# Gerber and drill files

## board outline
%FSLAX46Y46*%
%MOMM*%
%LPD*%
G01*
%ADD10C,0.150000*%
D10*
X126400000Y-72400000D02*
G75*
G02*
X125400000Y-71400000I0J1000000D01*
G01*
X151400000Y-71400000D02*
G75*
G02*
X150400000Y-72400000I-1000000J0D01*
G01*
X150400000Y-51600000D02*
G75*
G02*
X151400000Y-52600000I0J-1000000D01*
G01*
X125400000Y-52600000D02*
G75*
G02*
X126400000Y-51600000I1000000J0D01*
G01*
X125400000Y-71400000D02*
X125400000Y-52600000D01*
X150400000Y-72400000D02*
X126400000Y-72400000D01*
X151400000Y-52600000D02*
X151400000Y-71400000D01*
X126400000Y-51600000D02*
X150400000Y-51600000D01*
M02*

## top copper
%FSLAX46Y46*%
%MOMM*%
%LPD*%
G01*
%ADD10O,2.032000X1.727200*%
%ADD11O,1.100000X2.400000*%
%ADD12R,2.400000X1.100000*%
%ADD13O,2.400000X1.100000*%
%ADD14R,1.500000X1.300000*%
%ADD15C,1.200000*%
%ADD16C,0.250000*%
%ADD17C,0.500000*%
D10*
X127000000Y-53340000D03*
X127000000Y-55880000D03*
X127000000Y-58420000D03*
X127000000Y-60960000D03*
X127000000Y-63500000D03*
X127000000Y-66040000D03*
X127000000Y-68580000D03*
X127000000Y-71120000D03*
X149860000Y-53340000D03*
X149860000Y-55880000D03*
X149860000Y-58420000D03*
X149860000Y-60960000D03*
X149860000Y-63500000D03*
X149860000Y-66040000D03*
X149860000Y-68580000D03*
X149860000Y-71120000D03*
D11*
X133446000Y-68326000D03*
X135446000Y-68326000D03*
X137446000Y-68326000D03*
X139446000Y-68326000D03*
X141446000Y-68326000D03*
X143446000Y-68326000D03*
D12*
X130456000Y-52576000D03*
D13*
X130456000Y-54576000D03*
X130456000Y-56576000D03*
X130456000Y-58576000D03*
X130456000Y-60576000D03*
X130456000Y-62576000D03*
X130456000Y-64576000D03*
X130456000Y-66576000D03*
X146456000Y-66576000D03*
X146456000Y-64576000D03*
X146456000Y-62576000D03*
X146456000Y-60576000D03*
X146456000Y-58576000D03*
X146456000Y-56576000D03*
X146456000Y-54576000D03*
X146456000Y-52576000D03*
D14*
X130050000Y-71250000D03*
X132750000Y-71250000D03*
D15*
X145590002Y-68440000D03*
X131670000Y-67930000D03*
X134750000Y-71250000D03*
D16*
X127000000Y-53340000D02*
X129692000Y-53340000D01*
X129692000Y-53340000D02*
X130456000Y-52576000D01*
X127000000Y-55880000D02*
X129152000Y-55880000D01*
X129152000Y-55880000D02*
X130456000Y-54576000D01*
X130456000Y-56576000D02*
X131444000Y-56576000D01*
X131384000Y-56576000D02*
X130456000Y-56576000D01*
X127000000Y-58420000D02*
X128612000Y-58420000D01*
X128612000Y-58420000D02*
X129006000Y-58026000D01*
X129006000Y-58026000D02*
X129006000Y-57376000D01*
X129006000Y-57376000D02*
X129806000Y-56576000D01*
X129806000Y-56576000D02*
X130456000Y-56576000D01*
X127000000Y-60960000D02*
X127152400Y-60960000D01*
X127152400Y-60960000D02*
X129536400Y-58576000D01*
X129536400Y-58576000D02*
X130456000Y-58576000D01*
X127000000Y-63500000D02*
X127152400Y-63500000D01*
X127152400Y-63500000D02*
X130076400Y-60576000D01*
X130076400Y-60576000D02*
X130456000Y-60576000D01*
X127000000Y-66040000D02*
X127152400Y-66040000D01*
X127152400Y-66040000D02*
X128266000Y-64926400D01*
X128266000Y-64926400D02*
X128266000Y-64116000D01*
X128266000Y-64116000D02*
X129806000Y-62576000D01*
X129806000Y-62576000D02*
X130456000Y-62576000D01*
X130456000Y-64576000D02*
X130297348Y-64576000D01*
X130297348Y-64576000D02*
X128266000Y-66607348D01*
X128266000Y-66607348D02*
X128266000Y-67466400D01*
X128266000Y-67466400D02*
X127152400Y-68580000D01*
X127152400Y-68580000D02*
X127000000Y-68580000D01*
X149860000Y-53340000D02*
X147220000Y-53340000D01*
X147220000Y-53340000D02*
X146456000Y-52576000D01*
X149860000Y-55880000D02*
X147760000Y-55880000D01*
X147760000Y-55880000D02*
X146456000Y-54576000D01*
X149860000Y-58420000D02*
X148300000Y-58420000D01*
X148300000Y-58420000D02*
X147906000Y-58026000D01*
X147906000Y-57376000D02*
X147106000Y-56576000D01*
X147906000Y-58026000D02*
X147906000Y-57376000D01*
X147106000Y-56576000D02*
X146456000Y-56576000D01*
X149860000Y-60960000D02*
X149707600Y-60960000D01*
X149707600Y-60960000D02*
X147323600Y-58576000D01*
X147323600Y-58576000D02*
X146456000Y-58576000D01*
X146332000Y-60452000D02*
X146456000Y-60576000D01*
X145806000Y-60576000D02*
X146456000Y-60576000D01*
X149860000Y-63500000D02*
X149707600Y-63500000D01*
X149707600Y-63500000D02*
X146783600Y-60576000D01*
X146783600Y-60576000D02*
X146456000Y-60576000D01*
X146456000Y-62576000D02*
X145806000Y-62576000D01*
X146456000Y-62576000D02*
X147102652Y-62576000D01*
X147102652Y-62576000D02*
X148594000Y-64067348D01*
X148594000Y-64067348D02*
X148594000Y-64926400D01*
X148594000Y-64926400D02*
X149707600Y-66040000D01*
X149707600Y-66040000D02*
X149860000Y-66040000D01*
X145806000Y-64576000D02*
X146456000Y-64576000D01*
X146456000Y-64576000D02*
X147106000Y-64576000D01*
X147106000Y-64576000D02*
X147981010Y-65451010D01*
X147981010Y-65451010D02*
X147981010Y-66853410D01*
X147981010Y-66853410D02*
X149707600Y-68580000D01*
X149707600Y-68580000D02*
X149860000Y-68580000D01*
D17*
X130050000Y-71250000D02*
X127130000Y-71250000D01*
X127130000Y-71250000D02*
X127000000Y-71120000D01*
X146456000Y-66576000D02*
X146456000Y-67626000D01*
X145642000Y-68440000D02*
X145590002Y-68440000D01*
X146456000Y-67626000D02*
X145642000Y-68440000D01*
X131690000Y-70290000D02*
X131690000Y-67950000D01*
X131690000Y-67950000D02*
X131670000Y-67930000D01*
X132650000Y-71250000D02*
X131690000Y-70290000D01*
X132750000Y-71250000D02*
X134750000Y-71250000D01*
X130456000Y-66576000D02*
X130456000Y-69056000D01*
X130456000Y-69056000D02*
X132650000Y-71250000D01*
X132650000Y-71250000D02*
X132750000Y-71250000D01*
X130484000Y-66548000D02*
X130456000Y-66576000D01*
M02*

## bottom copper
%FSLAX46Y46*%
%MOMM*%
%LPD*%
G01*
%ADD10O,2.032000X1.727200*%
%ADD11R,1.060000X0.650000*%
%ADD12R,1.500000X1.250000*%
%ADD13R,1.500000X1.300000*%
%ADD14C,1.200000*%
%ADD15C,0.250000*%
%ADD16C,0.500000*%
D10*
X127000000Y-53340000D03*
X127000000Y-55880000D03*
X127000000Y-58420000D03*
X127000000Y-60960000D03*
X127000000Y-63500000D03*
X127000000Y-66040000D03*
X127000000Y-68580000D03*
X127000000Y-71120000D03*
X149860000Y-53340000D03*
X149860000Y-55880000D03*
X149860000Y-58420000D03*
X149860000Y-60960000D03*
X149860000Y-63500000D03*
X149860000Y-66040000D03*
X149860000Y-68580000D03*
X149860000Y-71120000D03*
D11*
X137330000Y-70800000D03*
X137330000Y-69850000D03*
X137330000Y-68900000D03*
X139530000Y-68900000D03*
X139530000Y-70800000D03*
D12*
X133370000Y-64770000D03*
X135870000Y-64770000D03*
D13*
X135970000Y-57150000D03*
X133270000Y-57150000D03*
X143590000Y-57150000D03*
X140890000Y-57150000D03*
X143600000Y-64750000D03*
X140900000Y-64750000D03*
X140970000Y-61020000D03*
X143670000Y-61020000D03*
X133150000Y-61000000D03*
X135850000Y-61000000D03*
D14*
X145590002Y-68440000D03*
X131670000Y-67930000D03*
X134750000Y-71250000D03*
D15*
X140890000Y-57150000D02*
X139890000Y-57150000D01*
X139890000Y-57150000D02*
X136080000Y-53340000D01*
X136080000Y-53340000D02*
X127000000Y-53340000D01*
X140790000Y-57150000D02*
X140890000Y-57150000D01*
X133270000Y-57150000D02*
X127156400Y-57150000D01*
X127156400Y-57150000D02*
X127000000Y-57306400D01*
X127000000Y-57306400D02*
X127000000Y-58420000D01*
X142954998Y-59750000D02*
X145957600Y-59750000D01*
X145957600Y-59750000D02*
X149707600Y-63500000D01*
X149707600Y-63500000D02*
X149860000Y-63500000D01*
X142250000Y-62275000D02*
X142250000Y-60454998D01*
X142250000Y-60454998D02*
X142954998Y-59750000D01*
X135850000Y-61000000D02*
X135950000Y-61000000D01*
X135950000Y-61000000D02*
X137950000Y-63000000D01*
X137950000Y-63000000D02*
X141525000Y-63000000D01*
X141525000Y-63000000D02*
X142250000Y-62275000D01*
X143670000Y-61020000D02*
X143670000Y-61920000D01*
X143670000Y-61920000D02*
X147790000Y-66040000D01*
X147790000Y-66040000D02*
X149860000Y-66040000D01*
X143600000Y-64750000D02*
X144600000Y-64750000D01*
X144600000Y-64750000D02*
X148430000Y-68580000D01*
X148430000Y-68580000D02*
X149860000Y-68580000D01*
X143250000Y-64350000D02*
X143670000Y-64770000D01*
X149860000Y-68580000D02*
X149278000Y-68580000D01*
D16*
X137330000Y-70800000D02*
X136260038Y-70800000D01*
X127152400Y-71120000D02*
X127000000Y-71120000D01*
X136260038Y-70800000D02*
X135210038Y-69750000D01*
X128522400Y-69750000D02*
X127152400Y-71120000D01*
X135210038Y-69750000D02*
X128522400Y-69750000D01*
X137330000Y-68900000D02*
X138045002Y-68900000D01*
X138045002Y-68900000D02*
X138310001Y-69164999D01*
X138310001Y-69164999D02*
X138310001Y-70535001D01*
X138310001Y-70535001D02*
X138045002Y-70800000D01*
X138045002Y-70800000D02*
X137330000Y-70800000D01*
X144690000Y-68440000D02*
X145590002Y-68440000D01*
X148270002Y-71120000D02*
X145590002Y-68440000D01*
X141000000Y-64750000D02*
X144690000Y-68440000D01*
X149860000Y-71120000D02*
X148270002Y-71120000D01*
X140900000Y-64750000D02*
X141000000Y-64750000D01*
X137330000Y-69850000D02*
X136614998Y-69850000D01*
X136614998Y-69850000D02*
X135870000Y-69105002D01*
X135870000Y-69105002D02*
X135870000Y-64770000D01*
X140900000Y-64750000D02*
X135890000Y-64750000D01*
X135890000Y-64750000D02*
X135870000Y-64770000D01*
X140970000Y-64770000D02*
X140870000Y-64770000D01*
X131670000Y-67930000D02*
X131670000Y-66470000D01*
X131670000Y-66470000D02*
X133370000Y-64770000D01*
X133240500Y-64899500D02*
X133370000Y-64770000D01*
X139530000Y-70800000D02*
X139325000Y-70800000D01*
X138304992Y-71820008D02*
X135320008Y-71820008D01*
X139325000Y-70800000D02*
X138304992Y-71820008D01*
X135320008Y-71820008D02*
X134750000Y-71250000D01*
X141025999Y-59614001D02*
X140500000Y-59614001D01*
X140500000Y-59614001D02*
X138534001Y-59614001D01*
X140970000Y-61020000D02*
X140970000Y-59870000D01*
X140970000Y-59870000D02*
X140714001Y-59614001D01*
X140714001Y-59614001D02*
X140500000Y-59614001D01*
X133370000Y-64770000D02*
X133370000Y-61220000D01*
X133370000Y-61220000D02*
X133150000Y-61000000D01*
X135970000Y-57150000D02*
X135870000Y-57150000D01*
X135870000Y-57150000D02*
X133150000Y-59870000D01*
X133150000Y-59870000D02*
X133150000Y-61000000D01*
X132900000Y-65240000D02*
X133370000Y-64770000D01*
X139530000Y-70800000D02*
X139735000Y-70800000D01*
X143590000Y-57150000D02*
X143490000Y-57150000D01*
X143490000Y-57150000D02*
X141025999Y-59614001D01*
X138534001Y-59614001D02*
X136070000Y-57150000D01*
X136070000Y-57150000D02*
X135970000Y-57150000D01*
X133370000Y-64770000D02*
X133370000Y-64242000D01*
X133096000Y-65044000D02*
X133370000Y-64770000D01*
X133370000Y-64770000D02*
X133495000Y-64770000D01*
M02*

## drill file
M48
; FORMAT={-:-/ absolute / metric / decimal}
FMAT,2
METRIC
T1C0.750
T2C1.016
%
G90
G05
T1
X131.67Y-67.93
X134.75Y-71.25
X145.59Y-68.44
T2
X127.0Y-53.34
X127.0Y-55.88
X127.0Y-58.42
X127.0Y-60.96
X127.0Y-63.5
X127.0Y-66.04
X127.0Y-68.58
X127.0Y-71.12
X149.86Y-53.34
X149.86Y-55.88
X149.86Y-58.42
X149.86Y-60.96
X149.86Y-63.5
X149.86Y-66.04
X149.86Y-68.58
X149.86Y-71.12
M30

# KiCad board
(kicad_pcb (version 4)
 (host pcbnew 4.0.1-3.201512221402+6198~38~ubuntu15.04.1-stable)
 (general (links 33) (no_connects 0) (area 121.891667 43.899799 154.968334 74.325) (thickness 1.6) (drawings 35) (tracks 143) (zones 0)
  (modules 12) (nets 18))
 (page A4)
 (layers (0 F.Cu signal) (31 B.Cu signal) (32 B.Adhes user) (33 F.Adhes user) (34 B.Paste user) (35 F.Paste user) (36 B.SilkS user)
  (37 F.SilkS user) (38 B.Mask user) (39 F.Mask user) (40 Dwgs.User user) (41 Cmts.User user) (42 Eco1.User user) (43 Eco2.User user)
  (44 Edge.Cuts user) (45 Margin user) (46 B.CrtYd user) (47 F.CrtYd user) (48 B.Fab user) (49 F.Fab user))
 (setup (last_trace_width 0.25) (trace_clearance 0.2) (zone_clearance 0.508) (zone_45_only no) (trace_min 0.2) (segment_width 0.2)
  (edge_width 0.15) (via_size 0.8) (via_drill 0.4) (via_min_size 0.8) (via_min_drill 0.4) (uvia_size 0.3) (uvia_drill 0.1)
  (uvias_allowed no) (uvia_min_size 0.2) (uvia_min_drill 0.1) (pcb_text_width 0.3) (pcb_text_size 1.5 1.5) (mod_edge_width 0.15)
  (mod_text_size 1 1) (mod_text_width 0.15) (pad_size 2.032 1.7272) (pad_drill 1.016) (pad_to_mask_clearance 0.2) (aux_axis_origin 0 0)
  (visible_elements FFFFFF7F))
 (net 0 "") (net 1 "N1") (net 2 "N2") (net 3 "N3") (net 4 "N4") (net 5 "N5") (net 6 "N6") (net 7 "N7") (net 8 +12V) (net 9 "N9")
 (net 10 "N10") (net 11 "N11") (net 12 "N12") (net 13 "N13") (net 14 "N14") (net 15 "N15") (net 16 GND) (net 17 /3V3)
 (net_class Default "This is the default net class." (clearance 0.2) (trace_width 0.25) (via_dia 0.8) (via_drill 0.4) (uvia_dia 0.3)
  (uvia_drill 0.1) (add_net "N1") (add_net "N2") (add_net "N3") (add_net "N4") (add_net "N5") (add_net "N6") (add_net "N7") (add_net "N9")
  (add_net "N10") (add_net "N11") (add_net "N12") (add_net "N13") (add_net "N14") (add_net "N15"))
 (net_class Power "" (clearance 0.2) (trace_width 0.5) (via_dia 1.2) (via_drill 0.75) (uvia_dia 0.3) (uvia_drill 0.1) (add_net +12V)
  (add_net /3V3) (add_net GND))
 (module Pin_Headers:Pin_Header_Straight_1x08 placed (layer B.Cu) (at 127 53.34 180)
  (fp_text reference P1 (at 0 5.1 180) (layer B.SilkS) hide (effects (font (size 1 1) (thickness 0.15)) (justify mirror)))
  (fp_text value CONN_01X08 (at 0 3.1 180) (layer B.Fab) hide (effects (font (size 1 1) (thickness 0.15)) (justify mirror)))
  (pad 1 thru_hole oval (at 0 0 180) (size 2.032 1.7272) (drill 1.016) (layers *.Cu *.Mask B.SilkS) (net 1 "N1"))
  (pad 2 thru_hole oval (at 0 -2.54 180) (size 2.032 1.7272) (drill 1.016) (layers *.Cu *.Mask B.SilkS) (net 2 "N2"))
  (pad 3 thru_hole oval (at 0 -5.08 180) (size 2.032 1.7272) (drill 1.016) (layers *.Cu *.Mask B.SilkS) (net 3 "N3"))
  (pad 4 thru_hole oval (at 0 -7.62 180) (size 2.032 1.7272) (drill 1.016) (layers *.Cu *.Mask B.SilkS) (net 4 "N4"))
  (pad 5 thru_hole oval (at 0 -10.16 180) (size 2.032 1.7272) (drill 1.016) (layers *.Cu *.Mask B.SilkS) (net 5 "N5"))
  (pad 6 thru_hole oval (at 0 -12.7 180) (size 2.032 1.7272) (drill 1.016) (layers *.Cu *.Mask B.SilkS) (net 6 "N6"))
  (pad 7 thru_hole oval (at 0 -15.24 180) (size 2.032 1.7272) (drill 1.016) (layers *.Cu *.Mask B.SilkS) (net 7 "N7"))
  (pad 8 thru_hole oval (at 0 -17.78 180) (size 2.032 1.7272) (drill 1.016) (layers *.Cu *.Mask B.SilkS) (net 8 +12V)))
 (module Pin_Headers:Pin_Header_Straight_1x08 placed (layer B.Cu) (at 149.86 53.34 180)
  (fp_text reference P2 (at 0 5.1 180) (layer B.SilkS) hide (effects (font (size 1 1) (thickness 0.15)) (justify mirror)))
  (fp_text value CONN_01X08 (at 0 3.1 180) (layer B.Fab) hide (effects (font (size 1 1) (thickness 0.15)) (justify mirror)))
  (pad 1 thru_hole oval (at 0 0 180) (size 2.032 1.7272) (drill 1.016) (layers *.Cu *.Mask B.SilkS) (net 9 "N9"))
  (pad 2 thru_hole oval (at 0 -2.54 180) (size 2.032 1.7272) (drill 1.016) (layers *.Cu *.Mask B.SilkS) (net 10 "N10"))
  (pad 3 thru_hole oval (at 0 -5.08 180) (size 2.032 1.7272) (drill 1.016) (layers *.Cu *.Mask B.SilkS) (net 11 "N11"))
  (pad 4 thru_hole oval (at 0 -7.62 180) (size 2.032 1.7272) (drill 1.016) (layers *.Cu *.Mask B.SilkS) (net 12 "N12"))
  (pad 5 thru_hole oval (at 0 -10.16 180) (size 2.032 1.7272) (drill 1.016) (layers *.Cu *.Mask B.SilkS) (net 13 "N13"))
  (pad 6 thru_hole oval (at 0 -12.7 180) (size 2.032 1.7272) (drill 1.016) (layers *.Cu *.Mask B.SilkS) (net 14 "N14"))
  (pad 7 thru_hole oval (at 0 -15.24 180) (size 2.032 1.7272) (drill 1.016) (layers *.Cu *.Mask B.SilkS) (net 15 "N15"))
  (pad 8 thru_hole oval (at 0 -17.78 180) (size 2.032 1.7272) (drill 1.016) (layers *.Cu *.Mask B.SilkS) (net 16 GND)))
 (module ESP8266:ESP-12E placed (layer F.Cu) (at 130.456 52.576)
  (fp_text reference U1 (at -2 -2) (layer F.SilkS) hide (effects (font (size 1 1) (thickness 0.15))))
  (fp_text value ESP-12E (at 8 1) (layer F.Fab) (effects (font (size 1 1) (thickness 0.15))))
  (pad 9 smd oval (at 2.99 15.75 90) (size 2.4 1.1) (layers F.Cu F.Paste F.Mask))
  (pad 10 smd oval (at 4.99 15.75 90) (size 2.4 1.1) (layers F.Cu F.Paste F.Mask))
  (pad 11 smd oval (at 6.99 15.75 90) (size 2.4 1.1) (layers F.Cu F.Paste F.Mask))
  (pad 12 smd oval (at 8.99 15.75 90) (size 2.4 1.1) (layers F.Cu F.Paste F.Mask))
  (pad 13 smd oval (at 10.99 15.75 90) (size 2.4 1.1) (layers F.Cu F.Paste F.Mask))
  (pad 14 smd oval (at 12.99 15.75 90) (size 2.4 1.1) (layers F.Cu F.Paste F.Mask))
  (pad 1 smd rect (at 0 0) (size 2.4 1.1) (layers F.Cu F.Paste F.Mask) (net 1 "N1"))
  (pad 2 smd oval (at 0 2) (size 2.4 1.1) (layers F.Cu F.Paste F.Mask) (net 2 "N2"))
  (pad 3 smd oval (at 0 4) (size 2.4 1.1) (layers F.Cu F.Paste F.Mask) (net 3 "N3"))
  (pad 4 smd oval (at 0 6) (size 2.4 1.1) (layers F.Cu F.Paste F.Mask) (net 4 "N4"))
  (pad 5 smd oval (at 0 8) (size 2.4 1.1) (layers F.Cu F.Paste F.Mask) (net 5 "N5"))
  (pad 6 smd oval (at 0 10) (size 2.4 1.1) (layers F.Cu F.Paste F.Mask) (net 6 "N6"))
  (pad 7 smd oval (at 0 12) (size 2.4 1.1) (layers F.Cu F.Paste F.Mask) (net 7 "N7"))
  (pad 8 smd oval (at 0 14) (size 2.4 1.1) (layers F.Cu F.Paste F.Mask) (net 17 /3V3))
  (pad 15 smd oval (at 16 14) (size 2.4 1.1) (layers F.Cu F.Paste F.Mask) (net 16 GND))
  (pad 16 smd oval (at 16 12) (size 2.4 1.1) (layers F.Cu F.Paste F.Mask) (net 15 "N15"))
  (pad 17 smd oval (at 16 10) (size 2.4 1.1) (layers F.Cu F.Paste F.Mask) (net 14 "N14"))
  (pad 18 smd oval (at 16 8) (size 2.4 1.1) (layers F.Cu F.Paste F.Mask) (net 13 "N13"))
  (pad 19 smd oval (at 16 6) (size 2.4 1.1) (layers F.Cu F.Paste F.Mask) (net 12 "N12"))
  (pad 20 smd oval (at 16 4) (size 2.4 1.1) (layers F.Cu F.Paste F.Mask) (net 11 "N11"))
  (pad 21 smd oval (at 16 2) (size 2.4 1.1) (layers F.Cu F.Paste F.Mask) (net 10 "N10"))
  (pad 22 smd oval (at 16 0) (size 2.4 1.1) (layers F.Cu F.Paste F.Mask) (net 9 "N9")))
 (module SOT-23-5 (layer B.Cu) (at 138.43 69.85)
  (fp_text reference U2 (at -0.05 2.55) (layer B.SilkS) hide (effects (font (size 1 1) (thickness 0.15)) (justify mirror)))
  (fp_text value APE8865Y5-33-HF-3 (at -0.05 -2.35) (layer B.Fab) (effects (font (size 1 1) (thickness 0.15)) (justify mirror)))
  (pad 1 smd rect (at -1.1 0.95) (size 1.06 0.65) (layers B.Cu B.Paste B.Mask) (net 8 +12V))
  (pad 2 smd rect (at -1.1 0) (size 1.06 0.65) (layers B.Cu B.Paste B.Mask) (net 16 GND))
  (pad 3 smd rect (at -1.1 -0.95) (size 1.06 0.65) (layers B.Cu B.Paste B.Mask) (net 8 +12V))
  (pad 4 smd rect (at 1.1 -0.95) (size 1.06 0.65) (layers B.Cu B.Paste B.Mask))
  (pad 5 smd rect (at 1.1 0.95) (size 1.06 0.65) (layers B.Cu B.Paste B.Mask) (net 17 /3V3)))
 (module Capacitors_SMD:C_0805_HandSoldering (layer B.Cu) (at 134.62 64.77)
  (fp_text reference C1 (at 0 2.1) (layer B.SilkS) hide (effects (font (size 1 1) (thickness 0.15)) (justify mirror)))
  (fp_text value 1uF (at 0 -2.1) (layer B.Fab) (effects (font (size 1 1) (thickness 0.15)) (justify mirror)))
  (pad 1 smd rect (at -1.25 0) (size 1.5 1.25) (layers B.Cu B.Paste B.Mask) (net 17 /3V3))
  (pad 2 smd rect (at 1.25 0) (size 1.5 1.25) (layers B.Cu B.Paste B.Mask) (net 16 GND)))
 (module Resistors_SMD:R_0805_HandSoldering (layer B.Cu) (at 134.62 57.15 180)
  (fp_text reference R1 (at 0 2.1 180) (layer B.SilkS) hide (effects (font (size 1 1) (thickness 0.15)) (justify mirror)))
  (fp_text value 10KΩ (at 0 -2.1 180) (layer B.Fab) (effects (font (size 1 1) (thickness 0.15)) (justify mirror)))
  (pad 1 smd rect (at -1.35 0 180) (size 1.5 1.3) (layers B.Cu B.Paste B.Mask) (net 17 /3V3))
  (pad 2 smd rect (at 1.35 0 180) (size 1.5 1.3) (layers B.Cu B.Paste B.Mask) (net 3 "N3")))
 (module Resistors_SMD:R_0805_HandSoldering (layer B.Cu) (at 142.24 57.15 180)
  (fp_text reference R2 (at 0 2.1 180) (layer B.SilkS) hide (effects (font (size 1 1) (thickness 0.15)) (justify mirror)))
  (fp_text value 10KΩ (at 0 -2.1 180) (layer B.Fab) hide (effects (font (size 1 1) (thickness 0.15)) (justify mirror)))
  (pad 1 smd rect (at -1.35 0 180) (size 1.5 1.3) (layers B.Cu B.Paste B.Mask) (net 17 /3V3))
  (pad 2 smd rect (at 1.35 0 180) (size 1.5 1.3) (layers B.Cu B.Paste B.Mask) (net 1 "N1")))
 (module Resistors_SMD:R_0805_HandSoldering (layer B.Cu) (at 142.25 64.75 180)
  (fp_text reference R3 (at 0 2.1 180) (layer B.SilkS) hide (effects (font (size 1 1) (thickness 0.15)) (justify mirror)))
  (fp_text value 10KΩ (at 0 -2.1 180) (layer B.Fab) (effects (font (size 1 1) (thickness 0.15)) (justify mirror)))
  (pad 1 smd rect (at -1.35 0 180) (size 1.5 1.3) (layers B.Cu B.Paste B.Mask) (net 15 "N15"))
  (pad 2 smd rect (at 1.35 0 180) (size 1.5 1.3) (layers B.Cu B.Paste B.Mask) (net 16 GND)))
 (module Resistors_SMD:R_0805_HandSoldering (layer B.Cu) (at 142.32 61.02)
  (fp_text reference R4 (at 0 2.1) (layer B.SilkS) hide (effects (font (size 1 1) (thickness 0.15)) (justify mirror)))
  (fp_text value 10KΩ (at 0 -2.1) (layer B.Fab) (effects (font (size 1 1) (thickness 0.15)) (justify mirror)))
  (pad 1 smd rect (at -1.35 0) (size 1.5 1.3) (layers B.Cu B.Paste B.Mask) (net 17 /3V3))
  (pad 2 smd rect (at 1.35 0) (size 1.5 1.3) (layers B.Cu B.Paste B.Mask) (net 14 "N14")))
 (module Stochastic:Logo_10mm (layer F.Cu) (at 138.5 59.5)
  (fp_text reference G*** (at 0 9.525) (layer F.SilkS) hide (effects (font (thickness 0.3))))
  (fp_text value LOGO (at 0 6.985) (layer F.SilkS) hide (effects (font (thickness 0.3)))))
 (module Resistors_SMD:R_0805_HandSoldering (layer F.Cu) (at 131.4 71.25)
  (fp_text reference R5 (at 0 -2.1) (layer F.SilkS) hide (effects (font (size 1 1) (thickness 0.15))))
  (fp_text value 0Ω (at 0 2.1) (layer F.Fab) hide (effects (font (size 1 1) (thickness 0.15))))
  (pad 1 smd rect (at -1.35 0) (size 1.5 1.3) (layers F.Cu F.Paste F.Mask) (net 8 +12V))
  (pad 2 smd rect (at 1.35 0) (size 1.5 1.3) (layers F.Cu F.Paste F.Mask) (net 17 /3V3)))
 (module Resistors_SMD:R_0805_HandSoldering (layer B.Cu) (at 134.5 61)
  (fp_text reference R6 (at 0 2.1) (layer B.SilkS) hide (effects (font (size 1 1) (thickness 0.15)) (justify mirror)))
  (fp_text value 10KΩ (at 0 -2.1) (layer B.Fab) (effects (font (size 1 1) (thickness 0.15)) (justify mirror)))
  (pad 1 smd rect (at -1.35 0) (size 1.5 1.3) (layers B.Cu B.Paste B.Mask) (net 17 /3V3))
  (pad 2 smd rect (at 1.35 0) (size 1.5 1.3) (layers B.Cu B.Paste B.Mask) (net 13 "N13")))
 (gr_arc (start 126.4 71.4) (end 126.4 72.4) (angle 90) (layer Edge.Cuts) (width 0.15))
 (gr_arc (start 150.4 71.4) (end 151.4 71.4) (angle 90) (layer Edge.Cuts) (width 0.15))
 (gr_arc (start 150.4 52.6) (end 150.4 51.6) (angle 90) (layer Edge.Cuts) (width 0.15))
 (gr_arc (start 126.4 52.6) (end 125.4 52.6) (angle 90) (layer Edge.Cuts) (width 0.15))
 (gr_line (start 125.4 71.4) (end 125.4 52.6) (layer Edge.Cuts) (width 0.15))
 (gr_line (start 150.4 72.4) (end 126.4 72.4) (layer Edge.Cuts) (width 0.15))
 (gr_line (start 151.4 52.6) (end 151.4 71.4) (layer Edge.Cuts) (width 0.15))
 (gr_line (start 126.4 51.6) (end 150.4 51.6) (layer Edge.Cuts) (width 0.15))
 (segment (start 140.89 57.15) (end 139.89 57.15) (width 0.25) (layer B.Cu) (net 1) (status 10))
 (segment (start 139.89 57.15) (end 136.08 53.34) (width 0.25) (layer B.Cu) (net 1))
 (segment (start 136.08 53.34) (end 127 53.34) (width 0.25) (layer B.Cu) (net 1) (status 20))
 (segment (start 140.79 57.15) (end 140.89 57.15) (width 0.25) (layer B.Cu) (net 1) (status 30))
 (segment (start 127 53.34) (end 129.692 53.34) (width 0.25) (layer F.Cu) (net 1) (status 10))
 (segment (start 129.692 53.34) (end 130.456 52.576) (width 0.25) (layer F.Cu) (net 1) (status 20))
 (segment (start 127 55.88) (end 129.152 55.88) (width 0.25) (layer F.Cu) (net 2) (status 10))
 (segment (start 129.152 55.88) (end 130.456 54.576) (width 0.25) (layer F.Cu) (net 2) (status 20))
 (segment (start 133.27 57.15) (end 127.1564 57.15) (width 0.25) (layer B.Cu) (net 3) (status 10))
 (segment (start 127.1564 57.15) (end 127 57.3064) (width 0.25) (layer B.Cu) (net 3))
 (segment (start 127 57.3064) (end 127 58.42) (width 0.25) (layer B.Cu) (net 3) (status 20))
 (segment (start 130.456 56.576) (end 131.444 56.576) (width 0.25) (layer F.Cu) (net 3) (status 30))
 (segment (start 131.384 56.576) (end 130.456 56.576) (width 0.25) (layer F.Cu) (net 3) (status 30))
 (segment (start 127 58.42) (end 128.612 58.42) (width 0.25) (layer F.Cu) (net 3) (status 10))
 (segment (start 128.612 58.42) (end 129.006 58.026) (width 0.25) (layer F.Cu) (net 3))
 (segment (start 129.006 58.026) (end 129.006 57.376) (width 0.25) (layer F.Cu) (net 3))
 (segment (start 129.006 57.376) (end 129.806 56.576) (width 0.25) (layer F.Cu) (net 3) (status 20))
 (segment (start 129.806 56.576) (end 130.456 56.576) (width 0.25) (layer F.Cu) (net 3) (status 30))
 (segment (start 127 60.96) (end 127.1524 60.96) (width 0.25) (layer F.Cu) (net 4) (status 30))
 (segment (start 127.1524 60.96) (end 129.5364 58.576) (width 0.25) (layer F.Cu) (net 4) (status 30))
 (segment (start 129.5364 58.576) (end 130.456 58.576) (width 0.25) (layer F.Cu) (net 4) (status 30))
 (segment (start 127 63.5) (end 127.1524 63.5) (width 0.25) (layer F.Cu) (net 5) (status 30))
 (segment (start 127.1524 63.5) (end 130.0764 60.576) (width 0.25) (layer F.Cu) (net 5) (status 30))
 (segment (start 130.0764 60.576) (end 130.456 60.576) (width 0.25) (layer F.Cu) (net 5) (status 30))
 (segment (start 127 66.04) (end 127.1524 66.04) (width 0.25) (layer F.Cu) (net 6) (status 30))
 (segment (start 127.1524 66.04) (end 128.266 64.9264) (width 0.25) (layer F.Cu) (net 6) (status 10))
 (segment (start 128.266 64.9264) (end 128.266 64.116) (width 0.25) (layer F.Cu) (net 6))
 (segment (start 128.266 64.116) (end 129.806 62.576) (width 0.25) (layer F.Cu) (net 6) (status 20))
 (segment (start 129.806 62.576) (end 130.456 62.576) (width 0.25) (layer F.Cu) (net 6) (status 30))
 (segment (start 130.456 64.576) (end 130.297348 64.576) (width 0.25) (layer F.Cu) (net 7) (status 30))
 (segment (start 130.297348 64.576) (end 128.266 66.607348) (width 0.25) (layer F.Cu) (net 7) (status 10))
 (segment (start 128.266 66.607348) (end 128.266 67.4664) (width 0.25) (layer F.Cu) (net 7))
 (segment (start 128.266 67.4664) (end 127.1524 68.58) (width 0.25) (layer F.Cu) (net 7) (status 20))
 (segment (start 127.1524 68.58) (end 127 68.58) (width 0.25) (layer F.Cu) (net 7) (status 30))
 (segment (start 149.86 53.34) (end 147.22 53.34) (width 0.25) (layer F.Cu) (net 9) (status 10))
 (segment (start 147.22 53.34) (end 146.456 52.576) (width 0.25) (layer F.Cu) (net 9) (status 20))
 (segment (start 149.86 55.88) (end 147.76 55.88) (width 0.25) (layer F.Cu) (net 10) (status 10))
 (segment (start 147.76 55.88) (end 146.456 54.576) (width 0.25) (layer F.Cu) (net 10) (status 20))
 (segment (start 149.86 58.42) (end 148.3 58.42) (width 0.25) (layer F.Cu) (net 11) (status 10))
 (segment (start 148.3 58.42) (end 147.906 58.026) (width 0.25) (layer F.Cu) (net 11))
 (segment (start 147.906 57.376) (end 147.106 56.576) (width 0.25) (layer F.Cu) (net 11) (status 20))
 (segment (start 147.906 58.026) (end 147.906 57.376) (width 0.25) (layer F.Cu) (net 11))
 (segment (start 147.106 56.576) (end 146.456 56.576) (width 0.25) (layer F.Cu) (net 11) (status 30))
 (segment (start 149.86 60.96) (end 149.7076 60.96) (width 0.25) (layer F.Cu) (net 12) (status 30))
 (segment (start 149.7076 60.96) (end 147.3236 58.576) (width 0.25) (layer F.Cu) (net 12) (status 30))
 (segment (start 147.3236 58.576) (end 146.456 58.576) (width 0.25) (layer F.Cu) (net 12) (status 30))
 (segment (start 142.954998 59.75) (end 145.9576 59.75) (width 0.25) (layer B.Cu) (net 13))
 (segment (start 145.9576 59.75) (end 149.7076 63.5) (width 0.25) (layer B.Cu) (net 13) (status 20))
 (segment (start 149.7076 63.5) (end 149.86 63.5) (width 0.25) (layer B.Cu) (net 13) (status 30))
 (segment (start 142.25 62.275) (end 142.25 60.454998) (width 0.25) (layer B.Cu) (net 13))
 (segment (start 142.25 60.454998) (end 142.954998 59.75) (width 0.25) (layer B.Cu) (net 13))
 (segment (start 135.85 61) (end 135.95 61) (width 0.25) (layer B.Cu) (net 13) (status 30))
 (segment (start 135.95 61) (end 137.95 63) (width 0.25) (layer B.Cu) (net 13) (status 10))
 (segment (start 137.95 63) (end 141.525 63) (width 0.25) (layer B.Cu) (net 13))
 (segment (start 141.525 63) (end 142.25 62.275) (width 0.25) (layer B.Cu) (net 13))
 (segment (start 146.332 60.452) (end 146.456 60.576) (width 0.25) (layer F.Cu) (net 13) (status 30))
 (segment (start 145.806 60.576) (end 146.456 60.576) (width 0.25) (layer F.Cu) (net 13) (status 30))
 (segment (start 149.86 63.5) (end 149.7076 63.5) (width 0.25) (layer F.Cu) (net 13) (status 30))
 (segment (start 149.7076 63.5) (end 146.7836 60.576) (width 0.25) (layer F.Cu) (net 13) (status 30))
 (segment (start 146.7836 60.576) (end 146.456 60.576) (width 0.25) (layer F.Cu) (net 13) (status 30))
 (segment (start 143.67 61.02) (end 143.67 61.92) (width 0.25) (layer B.Cu) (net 14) (status 10))
 (segment (start 143.67 61.92) (end 147.79 66.04) (width 0.25) (layer B.Cu) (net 14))
 (segment (start 147.79 66.04) (end 149.86 66.04) (width 0.25) (layer B.Cu) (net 14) (status 20))
 (segment (start 146.456 62.576) (end 145.806 62.576) (width 0.25) (layer F.Cu) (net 14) (status 30))
 (segment (start 146.456 62.576) (end 147.102652 62.576) (width 0.25) (layer F.Cu) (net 14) (status 30))
 (segment (start 147.102652 62.576) (end 148.594 64.067348) (width 0.25) (layer F.Cu) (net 14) (status 10))
 (segment (start 148.594 64.067348) (end 148.594 64.9264) (width 0.25) (layer F.Cu) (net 14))
 (segment (start 148.594 64.9264) (end 149.7076 66.04) (width 0.25) (layer F.Cu) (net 14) (status 20))
 (segment (start 149.7076 66.04) (end 149.86 66.04) (width 0.25) (layer F.Cu) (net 14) (status 30))
 (segment (start 143.6 64.75) (end 144.6 64.75) (width 0.25) (layer B.Cu) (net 15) (status 10))
 (segment (start 144.6 64.75) (end 148.43 68.58) (width 0.25) (layer B.Cu) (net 15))
 (segment (start 148.43 68.58) (end 149.86 68.58) (width 0.25) (layer B.Cu) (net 15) (status 20))
 (segment (start 143.25 64.35) (end 143.67 64.77) (width 0.25) (layer B.Cu) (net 15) (status 30))
 (segment (start 145.806 64.576) (end 146.456 64.576) (width 0.25) (layer F.Cu) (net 15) (status 30))
 (segment (start 149.86 68.58) (end 149.278 68.58) (width 0.25) (layer B.Cu) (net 15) (status 30))
 (segment (start 146.456 64.576) (end 147.106 64.576) (width 0.25) (layer F.Cu) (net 15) (status 30))
 (segment (start 147.106 64.576) (end 147.98101 65.45101) (width 0.25) (layer F.Cu) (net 15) (status 10))
 (segment (start 147.98101 65.45101) (end 147.98101 66.85341) (width 0.25) (layer F.Cu) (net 15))
 (segment (start 147.98101 66.85341) (end 149.7076 68.58) (width 0.25) (layer F.Cu) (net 15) (status 20))
 (segment (start 149.7076 68.58) (end 149.86 68.58) (width 0.25) (layer F.Cu) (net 15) (status 30))
 (segment (start 137.33 70.8) (end 136.260038 70.8) (width 0.5) (layer B.Cu) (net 8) (status 10))
 (segment (start 127.1524 71.12) (end 127 71.12) (width 0.5) (layer B.Cu) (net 8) (status 30))
 (segment (start 136.260038 70.8) (end 135.210038 69.75) (width 0.5) (layer B.Cu) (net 8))
 (segment (start 128.5224 69.75) (end 127.1524 71.12) (width 0.5) (layer B.Cu) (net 8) (status 20))
 (segment (start 135.210038 69.75) (end 128.5224 69.75) (width 0.5) (layer B.Cu) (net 8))
 (segment (start 137.33 68.9) (end 138.045002 68.9) (width 0.5) (layer B.Cu) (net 8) (status 10))
 (segment (start 138.045002 68.9) (end 138.310001 69.164999) (width 0.5) (layer B.Cu) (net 8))
 (segment (start 138.310001 69.164999) (end 138.310001 70.535001) (width 0.5) (layer B.Cu) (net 8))
 (segment (start 138.310001 70.535001) (end 138.045002 70.8) (width 0.5) (layer B.Cu) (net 8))
 (segment (start 138.045002 70.8) (end 137.33 70.8) (width 0.5) (layer B.Cu) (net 8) (status 20))
 (segment (start 130.05 71.25) (end 127.13 71.25) (width 0.5) (layer F.Cu) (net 8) (status 30))
 (segment (start 127.13 71.25) (end 127 71.12) (width 0.5) (layer F.Cu) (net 8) (status 30))
 (segment (start 144.69 68.44) (end 145.590002 68.44) (width 0.5) (layer B.Cu) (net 16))
 (segment (start 146.456 66.576) (end 146.456 67.626) (width 0.5) (layer F.Cu) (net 16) (status 10))
 (segment (start 148.270002 71.12) (end 145.590002 68.44) (width 0.5) (layer B.Cu) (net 16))
 (segment (start 141 64.75) (end 144.69 68.44) (width 0.5) (layer B.Cu) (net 16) (status 10))
 (segment (start 145.642 68.44) (end 145.590002 68.44) (width 0.5) (layer F.Cu) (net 16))
 (segment (start 149.86 71.12) (end 148.270002 71.12) (width 0.5) (layer B.Cu) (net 16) (status 10))
 (segment (start 146.456 67.626) (end 145.642 68.44) (width 0.5) (layer F.Cu) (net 16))
 (segment (start 140.9 64.75) (end 141 64.75) (width 0.5) (layer B.Cu) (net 16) (status 30))
 (via (at 145.590002 68.44) (size 1.2) (drill 0.75) (layers F.Cu B.Cu) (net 16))
 (segment (start 137.33 69.85) (end 136.614998 69.85) (width 0.5) (layer B.Cu) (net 16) (status 10))
 (segment (start 136.614998 69.85) (end 135.87 69.105002) (width 0.5) (layer B.Cu) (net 16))
 (segment (start 135.87 69.105002) (end 135.87 64.77) (width 0.5) (layer B.Cu) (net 16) (status 20))
 (segment (start 140.9 64.75) (end 135.89 64.75) (width 0.5) (layer B.Cu) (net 16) (status 30))
 (segment (start 135.89 64.75) (end 135.87 64.77) (width 0.5) (layer B.Cu) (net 16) (status 30))
 (segment (start 140.97 64.77) (end 140.87 64.77) (width 0.5) (layer B.Cu) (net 16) (status 30))
 (segment (start 131.67 67.93) (end 131.67 66.47) (width 0.5) (layer B.Cu) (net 17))
 (segment (start 131.67 66.47) (end 133.37 64.77) (width 0.5) (layer B.Cu) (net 17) (status 20))
 (segment (start 131.69 70.29) (end 131.69 67.95) (width 0.5) (layer F.Cu) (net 17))
 (segment (start 131.69 67.95) (end 131.67 67.93) (width 0.5) (layer F.Cu) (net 17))
 (via (at 131.67 67.93) (size 1.2) (drill 0.75) (layers F.Cu B.Cu) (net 17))
 (segment (start 132.65 71.25) (end 131.69 70.29) (width 0.5) (layer F.Cu) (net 17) (status 10))
 (segment (start 133.2405 64.8995) (end 133.37 64.77) (width 0.5) (layer B.Cu) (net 17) (status 30))
 (via (at 134.75 71.25) (size 1.2) (drill 0.75) (layers F.Cu B.Cu) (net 17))
 (segment (start 132.75 71.25) (end 134.75 71.25) (width 0.5) (layer F.Cu) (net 17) (status 10))
 (segment (start 139.53 70.8) (end 139.325 70.8) (width 0.5) (layer B.Cu) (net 17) (status 30))
 (segment (start 138.304992 71.820008) (end 135.320008 71.820008) (width 0.5) (layer B.Cu) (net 17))
 (segment (start 139.325 70.8) (end 138.304992 71.820008) (width 0.5) (layer B.Cu) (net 17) (status 10))
 (segment (start 135.320008 71.820008) (end 134.75 71.25) (width 0.5) (layer B.Cu) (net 17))
 (segment (start 141.025999 59.614001) (end 140.5 59.614001) (width 0.5) (layer B.Cu) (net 17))
 (segment (start 140.5 59.614001) (end 138.534001 59.614001) (width 0.5) (layer B.Cu) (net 17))
 (segment (start 140.97 61.02) (end 140.97 59.87) (width 0.5) (layer B.Cu) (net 17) (status 10))
 (segment (start 140.97 59.87) (end 140.714001 59.614001) (width 0.5) (layer B.Cu) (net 17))
 (segment (start 140.714001 59.614001) (end 140.5 59.614001) (width 0.5) (layer B.Cu) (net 17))
 (segment (start 133.37 64.77) (end 133.37 61.22) (width 0.5) (layer B.Cu) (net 17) (status 30))
 (segment (start 133.37 61.22) (end 133.15 61) (width 0.5) (layer B.Cu) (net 17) (status 30))
 (segment (start 135.97 57.15) (end 135.87 57.15) (width 0.5) (layer B.Cu) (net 17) (status 30))
 (segment (start 135.87 57.15) (end 133.15 59.87) (width 0.5) (layer B.Cu) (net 17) (status 10))
 (segment (start 133.15 59.87) (end 133.15 61) (width 0.5) (layer B.Cu) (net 17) (status 20))
 (segment (start 132.9 65.24) (end 133.37 64.77) (width 0.5) (layer B.Cu) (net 17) (status 30))
 (segment (start 130.456 66.576) (end 130.456 69.056) (width 0.5) (layer F.Cu) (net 17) (status 10))
 (segment (start 130.456 69.056) (end 132.65 71.25) (width 0.5) (layer F.Cu) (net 17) (status 20))
 (segment (start 132.65 71.25) (end 132.75 71.25) (width 0.5) (layer F.Cu) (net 17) (status 30))
 (segment (start 139.53 70.8) (end 139.735 70.8) (width 0.5) (layer B.Cu) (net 17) (status 30))
 (segment (start 143.59 57.15) (end 143.49 57.15) (width 0.5) (layer B.Cu) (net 17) (status 30))
 (segment (start 143.49 57.15) (end 141.025999 59.614001) (width 0.5) (layer B.Cu) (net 17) (status 10))
 (segment (start 138.534001 59.614001) (end 136.07 57.15) (width 0.5) (layer B.Cu) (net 17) (status 20))
 (segment (start 136.07 57.15) (end 135.97 57.15) (width 0.5) (layer B.Cu) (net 17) (status 30))
 (segment (start 130.484 66.548) (end 130.456 66.576) (width 0.5) (layer F.Cu) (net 17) (status 30))
 (segment (start 133.37 64.77) (end 133.37 64.242) (width 0.5) (layer B.Cu) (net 17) (status 30))
 (segment (start 133.096 65.044) (end 133.37 64.77) (width 0.5) (layer B.Cu) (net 17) (status 30))
 (segment (start 133.37 64.77) (end 133.495 64.77) (width 0.5) (layer B.Cu) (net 17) (status 30)))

